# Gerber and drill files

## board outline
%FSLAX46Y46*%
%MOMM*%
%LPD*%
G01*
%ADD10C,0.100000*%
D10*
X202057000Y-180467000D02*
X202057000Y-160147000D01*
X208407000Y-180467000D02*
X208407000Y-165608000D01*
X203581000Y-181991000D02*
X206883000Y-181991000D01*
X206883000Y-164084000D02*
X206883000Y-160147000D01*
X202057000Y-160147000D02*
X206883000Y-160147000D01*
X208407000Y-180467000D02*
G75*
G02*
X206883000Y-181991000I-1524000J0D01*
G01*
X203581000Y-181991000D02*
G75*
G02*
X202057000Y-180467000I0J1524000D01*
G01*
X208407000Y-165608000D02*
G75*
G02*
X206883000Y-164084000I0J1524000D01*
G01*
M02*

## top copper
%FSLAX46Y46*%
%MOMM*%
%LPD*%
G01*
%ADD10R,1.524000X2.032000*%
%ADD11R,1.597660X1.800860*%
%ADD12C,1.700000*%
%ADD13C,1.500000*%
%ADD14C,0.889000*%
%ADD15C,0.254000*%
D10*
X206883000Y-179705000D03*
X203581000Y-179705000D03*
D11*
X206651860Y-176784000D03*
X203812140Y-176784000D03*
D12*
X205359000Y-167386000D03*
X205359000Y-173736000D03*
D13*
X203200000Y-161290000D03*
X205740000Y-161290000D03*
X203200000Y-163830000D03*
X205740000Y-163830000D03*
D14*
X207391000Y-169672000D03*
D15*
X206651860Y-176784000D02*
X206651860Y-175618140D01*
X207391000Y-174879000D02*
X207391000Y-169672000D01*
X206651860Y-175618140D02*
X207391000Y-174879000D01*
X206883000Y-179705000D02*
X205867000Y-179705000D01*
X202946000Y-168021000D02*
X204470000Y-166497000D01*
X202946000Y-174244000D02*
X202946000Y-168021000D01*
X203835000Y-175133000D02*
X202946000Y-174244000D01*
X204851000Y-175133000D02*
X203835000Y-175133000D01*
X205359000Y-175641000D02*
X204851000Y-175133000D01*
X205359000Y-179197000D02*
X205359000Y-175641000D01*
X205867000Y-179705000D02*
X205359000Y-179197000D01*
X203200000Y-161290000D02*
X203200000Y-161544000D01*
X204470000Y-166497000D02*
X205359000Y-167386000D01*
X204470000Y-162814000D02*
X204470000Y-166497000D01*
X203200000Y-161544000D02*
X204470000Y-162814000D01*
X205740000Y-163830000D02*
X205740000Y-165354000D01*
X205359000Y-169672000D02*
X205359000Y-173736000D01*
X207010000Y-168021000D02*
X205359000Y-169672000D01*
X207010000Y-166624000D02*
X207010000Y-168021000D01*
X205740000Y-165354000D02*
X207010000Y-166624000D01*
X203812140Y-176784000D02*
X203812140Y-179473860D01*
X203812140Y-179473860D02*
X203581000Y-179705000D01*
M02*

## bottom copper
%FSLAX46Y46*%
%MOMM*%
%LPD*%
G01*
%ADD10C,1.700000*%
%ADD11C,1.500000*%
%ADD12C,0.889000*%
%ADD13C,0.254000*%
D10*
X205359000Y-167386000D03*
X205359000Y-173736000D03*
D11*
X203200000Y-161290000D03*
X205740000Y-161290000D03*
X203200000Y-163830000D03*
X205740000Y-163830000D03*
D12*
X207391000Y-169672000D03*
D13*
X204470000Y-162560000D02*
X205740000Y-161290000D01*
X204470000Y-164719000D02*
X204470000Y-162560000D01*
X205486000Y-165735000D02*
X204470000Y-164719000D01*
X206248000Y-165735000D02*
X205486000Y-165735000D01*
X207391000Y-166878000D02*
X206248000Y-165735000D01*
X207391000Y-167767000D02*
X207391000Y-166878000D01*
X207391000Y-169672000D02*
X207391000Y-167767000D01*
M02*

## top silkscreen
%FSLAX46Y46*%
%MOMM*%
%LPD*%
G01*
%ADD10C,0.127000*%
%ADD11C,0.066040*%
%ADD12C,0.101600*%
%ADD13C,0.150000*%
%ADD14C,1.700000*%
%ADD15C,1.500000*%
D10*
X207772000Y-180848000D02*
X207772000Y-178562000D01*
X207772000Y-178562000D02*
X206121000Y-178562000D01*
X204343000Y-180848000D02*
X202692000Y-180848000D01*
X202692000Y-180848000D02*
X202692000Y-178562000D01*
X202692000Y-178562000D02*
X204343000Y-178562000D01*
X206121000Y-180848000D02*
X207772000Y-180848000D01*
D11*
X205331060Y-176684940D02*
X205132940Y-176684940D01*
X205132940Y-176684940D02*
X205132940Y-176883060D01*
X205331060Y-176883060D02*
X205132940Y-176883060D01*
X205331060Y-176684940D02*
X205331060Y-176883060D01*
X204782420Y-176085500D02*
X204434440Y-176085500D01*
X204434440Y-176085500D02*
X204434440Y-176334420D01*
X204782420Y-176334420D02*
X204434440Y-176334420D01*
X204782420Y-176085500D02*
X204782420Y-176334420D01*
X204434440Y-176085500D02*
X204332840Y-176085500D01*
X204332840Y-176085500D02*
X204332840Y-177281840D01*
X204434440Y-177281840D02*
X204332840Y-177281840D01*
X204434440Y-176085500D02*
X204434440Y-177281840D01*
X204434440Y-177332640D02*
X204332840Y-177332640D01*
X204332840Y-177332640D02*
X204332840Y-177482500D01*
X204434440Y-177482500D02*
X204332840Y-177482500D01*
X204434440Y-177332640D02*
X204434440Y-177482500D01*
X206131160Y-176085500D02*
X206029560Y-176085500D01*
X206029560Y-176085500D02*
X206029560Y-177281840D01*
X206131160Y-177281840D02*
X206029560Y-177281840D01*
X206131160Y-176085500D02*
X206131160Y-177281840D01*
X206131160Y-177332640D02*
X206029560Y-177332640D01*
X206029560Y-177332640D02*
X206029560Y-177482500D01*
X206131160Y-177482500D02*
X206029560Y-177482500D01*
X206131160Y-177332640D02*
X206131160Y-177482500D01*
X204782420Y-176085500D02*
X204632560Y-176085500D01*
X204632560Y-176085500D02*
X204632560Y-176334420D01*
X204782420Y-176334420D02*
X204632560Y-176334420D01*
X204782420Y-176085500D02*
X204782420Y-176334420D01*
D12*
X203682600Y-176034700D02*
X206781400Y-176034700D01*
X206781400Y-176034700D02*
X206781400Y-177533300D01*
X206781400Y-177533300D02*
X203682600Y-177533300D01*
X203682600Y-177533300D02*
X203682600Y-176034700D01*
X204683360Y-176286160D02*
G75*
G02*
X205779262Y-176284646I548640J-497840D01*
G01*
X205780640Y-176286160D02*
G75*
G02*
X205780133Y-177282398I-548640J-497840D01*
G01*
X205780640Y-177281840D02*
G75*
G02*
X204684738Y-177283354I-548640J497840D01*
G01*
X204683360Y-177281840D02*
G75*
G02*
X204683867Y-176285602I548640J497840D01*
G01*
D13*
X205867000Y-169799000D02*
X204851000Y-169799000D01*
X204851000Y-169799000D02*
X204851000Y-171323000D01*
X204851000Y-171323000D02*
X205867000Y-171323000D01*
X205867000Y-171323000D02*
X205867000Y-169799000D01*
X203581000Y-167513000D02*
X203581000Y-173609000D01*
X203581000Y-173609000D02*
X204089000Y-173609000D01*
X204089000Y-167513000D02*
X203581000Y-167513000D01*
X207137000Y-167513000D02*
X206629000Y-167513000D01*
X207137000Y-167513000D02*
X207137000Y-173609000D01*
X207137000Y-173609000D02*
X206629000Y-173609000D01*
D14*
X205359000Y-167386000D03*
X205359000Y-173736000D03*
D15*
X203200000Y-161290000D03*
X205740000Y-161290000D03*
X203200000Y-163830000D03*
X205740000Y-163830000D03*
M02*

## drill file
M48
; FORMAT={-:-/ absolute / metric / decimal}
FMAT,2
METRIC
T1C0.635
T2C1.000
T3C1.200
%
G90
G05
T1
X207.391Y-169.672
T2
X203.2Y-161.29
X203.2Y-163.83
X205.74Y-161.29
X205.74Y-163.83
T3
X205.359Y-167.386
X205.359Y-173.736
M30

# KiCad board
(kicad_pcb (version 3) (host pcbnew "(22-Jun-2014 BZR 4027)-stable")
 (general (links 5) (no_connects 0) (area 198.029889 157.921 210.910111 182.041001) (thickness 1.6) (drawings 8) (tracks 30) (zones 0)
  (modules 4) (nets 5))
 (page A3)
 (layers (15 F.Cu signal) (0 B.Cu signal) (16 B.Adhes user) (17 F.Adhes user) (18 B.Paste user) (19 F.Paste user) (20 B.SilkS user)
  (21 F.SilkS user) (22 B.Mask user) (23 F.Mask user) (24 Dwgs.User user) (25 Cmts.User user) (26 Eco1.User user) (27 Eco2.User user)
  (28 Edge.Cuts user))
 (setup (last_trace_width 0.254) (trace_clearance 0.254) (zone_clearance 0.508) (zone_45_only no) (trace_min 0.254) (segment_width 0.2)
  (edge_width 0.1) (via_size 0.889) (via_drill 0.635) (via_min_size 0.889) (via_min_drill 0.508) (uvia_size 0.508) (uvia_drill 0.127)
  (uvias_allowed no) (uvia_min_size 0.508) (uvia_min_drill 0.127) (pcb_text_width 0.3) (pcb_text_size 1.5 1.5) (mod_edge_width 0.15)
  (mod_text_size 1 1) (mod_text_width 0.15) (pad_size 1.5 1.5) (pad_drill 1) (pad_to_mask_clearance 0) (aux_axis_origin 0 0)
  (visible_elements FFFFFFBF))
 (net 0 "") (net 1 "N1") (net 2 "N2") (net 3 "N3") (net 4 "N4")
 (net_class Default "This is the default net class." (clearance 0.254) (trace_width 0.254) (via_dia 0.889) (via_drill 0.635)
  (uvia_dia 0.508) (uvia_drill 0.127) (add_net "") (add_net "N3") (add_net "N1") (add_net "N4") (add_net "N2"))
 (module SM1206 (layer F.Cu) (at 205.232 179.705 180)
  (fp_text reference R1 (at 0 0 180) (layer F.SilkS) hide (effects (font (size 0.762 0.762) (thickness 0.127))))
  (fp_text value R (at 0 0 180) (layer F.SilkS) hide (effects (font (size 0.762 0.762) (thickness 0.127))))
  (fp_line (start -2.54 -1.143) (end -2.54 1.143) (layer F.SilkS) (width 0.127))
  (fp_line (start -2.54 1.143) (end -0.889 1.143) (layer F.SilkS) (width 0.127))
  (fp_line (start 0.889 -1.143) (end 2.54 -1.143) (layer F.SilkS) (width 0.127))
  (fp_line (start 2.54 -1.143) (end 2.54 1.143) (layer F.SilkS) (width 0.127))
  (fp_line (start 2.54 1.143) (end 0.889 1.143) (layer F.SilkS) (width 0.127))
  (fp_line (start -0.889 -1.143) (end -2.54 -1.143) (layer F.SilkS) (width 0.127))
  (pad 1 smd rect (at -1.651 0 180) (size 1.524 2.032) (layers F.Cu F.Paste F.Mask) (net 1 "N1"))
  (pad 2 smd rect (at 1.651 0 180) (size 1.524 2.032) (layers F.Cu F.Paste F.Mask) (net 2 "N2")))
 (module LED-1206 (layer F.Cu) (at 205.232 176.784 180)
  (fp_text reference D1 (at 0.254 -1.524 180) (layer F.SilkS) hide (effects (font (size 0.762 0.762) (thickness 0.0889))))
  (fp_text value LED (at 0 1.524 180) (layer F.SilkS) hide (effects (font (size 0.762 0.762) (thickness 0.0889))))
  (fp_line (start -0.09906 0.09906) (end 0.09906 0.09906) (layer F.SilkS) (width 0.06604))
  (fp_line (start 0.09906 0.09906) (end 0.09906 -0.09906) (layer F.SilkS) (width 0.06604))
  (fp_line (start -0.09906 -0.09906) (end 0.09906 -0.09906) (layer F.SilkS) (width 0.06604))
  (fp_line (start -0.09906 0.09906) (end -0.09906 -0.09906) (layer F.SilkS) (width 0.06604))
  (fp_line (start 0.44958 0.6985) (end 0.79756 0.6985) (layer F.SilkS) (width 0.06604))
  (fp_line (start 0.79756 0.6985) (end 0.79756 0.44958) (layer F.SilkS) (width 0.06604))
  (fp_line (start 0.44958 0.44958) (end 0.79756 0.44958) (layer F.SilkS) (width 0.06604))
  (fp_line (start 0.44958 0.6985) (end 0.44958 0.44958) (layer F.SilkS) (width 0.06604))
  (fp_line (start 0.79756 0.6985) (end 0.89916 0.6985) (layer F.SilkS) (width 0.06604))
  (fp_line (start 0.89916 0.6985) (end 0.89916 -0.49784) (layer F.SilkS) (width 0.06604))
  (fp_line (start 0.79756 -0.49784) (end 0.89916 -0.49784) (layer F.SilkS) (width 0.06604))
  (fp_line (start 0.79756 0.6985) (end 0.79756 -0.49784) (layer F.SilkS) (width 0.06604))
  (fp_line (start 0.79756 -0.54864) (end 0.89916 -0.54864) (layer F.SilkS) (width 0.06604))
  (fp_line (start 0.89916 -0.54864) (end 0.89916 -0.6985) (layer F.SilkS) (width 0.06604))
  (fp_line (start 0.79756 -0.6985) (end 0.89916 -0.6985) (layer F.SilkS) (width 0.06604))
  (fp_line (start 0.79756 -0.54864) (end 0.79756 -0.6985) (layer F.SilkS) (width 0.06604))
  (fp_line (start -0.89916 0.6985) (end -0.79756 0.6985) (layer F.SilkS) (width 0.06604))
  (fp_line (start -0.79756 0.6985) (end -0.79756 -0.49784) (layer F.SilkS) (width 0.06604))
  (fp_line (start -0.89916 -0.49784) (end -0.79756 -0.49784) (layer F.SilkS) (width 0.06604))
  (fp_line (start -0.89916 0.6985) (end -0.89916 -0.49784) (layer F.SilkS) (width 0.06604))
  (fp_line (start -0.89916 -0.54864) (end -0.79756 -0.54864) (layer F.SilkS) (width 0.06604))
  (fp_line (start -0.79756 -0.54864) (end -0.79756 -0.6985) (layer F.SilkS) (width 0.06604))
  (fp_line (start -0.89916 -0.6985) (end -0.79756 -0.6985) (layer F.SilkS) (width 0.06604))
  (fp_line (start -0.89916 -0.54864) (end -0.89916 -0.6985) (layer F.SilkS) (width 0.06604))
  (fp_line (start 0.44958 0.6985) (end 0.59944 0.6985) (layer F.SilkS) (width 0.06604))
  (fp_line (start 0.59944 0.6985) (end 0.59944 0.44958) (layer F.SilkS) (width 0.06604))
  (fp_line (start 0.44958 0.44958) (end 0.59944 0.44958) (layer F.SilkS) (width 0.06604))
  (fp_line (start 0.44958 0.6985) (end 0.44958 0.44958) (layer F.SilkS) (width 0.06604))
  (fp_line (start 1.5494 0.7493) (end -1.5494 0.7493) (layer F.SilkS) (width 0.1016))
  (fp_line (start -1.5494 0.7493) (end -1.5494 -0.7493) (layer F.SilkS) (width 0.1016))
  (fp_line (start -1.5494 -0.7493) (end 1.5494 -0.7493) (layer F.SilkS) (width 0.1016))
  (fp_line (start 1.5494 -0.7493) (end 1.5494 0.7493) (layer F.SilkS) (width 0.1016))
  (fp_arc (start 0 0) (end 0.54864 0.49784) (angle 95.4) (layer F.SilkS) (width 0.1016))
  (fp_arc (start 0 0) (end -0.54864 0.49784) (angle 84.5) (layer F.SilkS) (width 0.1016))
  (fp_arc (start 0 0) (end -0.54864 -0.49784) (angle 95.4) (layer F.SilkS) (width 0.1016))
  (fp_arc (start 0 0) (end 0.54864 -0.49784) (angle 84.5) (layer F.SilkS) (width 0.1016))
  (pad 1 smd rect (at -1.41986 0 180) (size 1.59766 1.80086) (layers F.Cu F.Paste F.Mask) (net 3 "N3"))
  (pad 2 smd rect (at 1.41986 0 180) (size 1.59766 1.80086) (layers F.Cu F.Paste F.Mask) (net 2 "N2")))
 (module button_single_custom (layer F.Cu) (at 205.359 170.561 270)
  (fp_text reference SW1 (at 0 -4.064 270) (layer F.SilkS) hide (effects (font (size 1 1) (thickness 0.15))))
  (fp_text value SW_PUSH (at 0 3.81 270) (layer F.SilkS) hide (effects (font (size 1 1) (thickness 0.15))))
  (fp_line (start -0.762 -0.508) (end -0.762 0.508) (layer F.SilkS) (width 0.15))
  (fp_line (start -0.762 0.508) (end 0.762 0.508) (layer F.SilkS) (width 0.15))
  (fp_line (start 0.762 0.508) (end 0.762 -0.508) (layer F.SilkS) (width 0.15))
  (fp_line (start 0.762 -0.508) (end -0.762 -0.508) (layer F.SilkS) (width 0.15))
  (fp_line (start -3.048 1.778) (end 3.048 1.778) (layer F.SilkS) (width 0.15))
  (fp_line (start 3.048 1.778) (end 3.048 1.27) (layer F.SilkS) (width 0.15))
  (fp_line (start -3.048 1.27) (end -3.048 1.778) (layer F.SilkS) (width 0.15))
  (fp_line (start -3.048 -1.778) (end -3.048 -1.27) (layer F.SilkS) (width 0.15))
  (fp_line (start -3.048 -1.778) (end 3.048 -1.778) (layer F.SilkS) (width 0.15))
  (fp_line (start 3.048 -1.778) (end 3.048 -1.27) (layer F.SilkS) (width 0.15))
  (pad 1 thru_hole circle (at -3.175 0 270) (size 1.7 1.7) (drill 1.2) (layers *.Cu *.Mask F.SilkS) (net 1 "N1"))
  (pad 2 thru_hole circle (at 3.175 0 270) (size 1.7 1.7) (drill 1.2) (layers *.Cu *.Mask F.SilkS) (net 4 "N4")))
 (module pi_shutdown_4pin (layer F.Cu) (at 204.47 162.56)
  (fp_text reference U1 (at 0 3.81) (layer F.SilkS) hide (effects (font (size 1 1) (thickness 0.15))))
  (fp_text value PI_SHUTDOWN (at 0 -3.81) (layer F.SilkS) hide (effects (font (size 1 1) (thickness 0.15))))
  (pad 14 thru_hole circle (at -1.27 -1.27) (size 1.5 1.5) (drill 1) (layers *.Cu *.Mask F.SilkS) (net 1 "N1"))
  (pad 16 thru_hole circle (at 1.27 -1.27) (size 1.5 1.5) (drill 1) (layers *.Cu *.Mask F.SilkS) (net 3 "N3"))
  (pad 13 thru_hole circle (at -1.27 1.27) (size 1.5 1.5) (drill 1) (layers *.Cu *.Mask F.SilkS))
  (pad 15 thru_hole circle (at 1.27 1.27) (size 1.5 1.5) (drill 1) (layers *.Cu *.Mask F.SilkS) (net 4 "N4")))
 (gr_line (start 202.057 180.467) (end 202.057 160.147) (angle 90) (layer Edge.Cuts) (width 0.1))
 (gr_line (start 208.407 180.467) (end 208.407 165.608) (angle 90) (layer Edge.Cuts) (width 0.1))
 (gr_line (start 203.581 181.991) (end 206.883 181.991) (angle 90) (layer Edge.Cuts) (width 0.1))
 (gr_line (start 206.883 164.084) (end 206.883 160.147) (angle 90) (layer Edge.Cuts) (width 0.1))
 (gr_line (start 202.057 160.147) (end 206.883 160.147) (angle 90) (layer Edge.Cuts) (width 0.1))
 (gr_arc (start 206.883 180.467) (end 208.407 180.467) (angle 90) (layer Edge.Cuts) (width 0.1))
 (gr_arc (start 203.581 180.467) (end 203.581 181.991) (angle 90) (layer Edge.Cuts) (width 0.1))
 (gr_arc (start 208.407 164.084) (end 208.407 165.608) (angle 90) (layer Edge.Cuts) (width 0.1))
 (segment (start 206.65186 176.784) (end 206.65186 175.61814) (width 0.254) (layer F.Cu) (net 3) (status 400000))
 (segment (start 204.47 162.56) (end 205.74 161.29) (width 0.254) (layer B.Cu) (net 3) (status 800000))
 (segment (start 204.47 164.719) (end 204.47 162.56) (width 0.254) (layer B.Cu) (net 3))
 (segment (start 205.486 165.735) (end 204.47 164.719) (width 0.254) (layer B.Cu) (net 3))
 (segment (start 206.248 165.735) (end 205.486 165.735) (width 0.254) (layer B.Cu) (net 3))
 (segment (start 207.391 166.878) (end 206.248 165.735) (width 0.254) (layer B.Cu) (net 3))
 (segment (start 207.391 167.767) (end 207.391 166.878) (width 0.254) (layer B.Cu) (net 3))
 (segment (start 207.391 169.672) (end 207.391 167.767) (width 0.254) (layer B.Cu) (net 3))
 (segment (start 207.391 174.879) (end 207.391 169.672) (width 0.254) (layer F.Cu) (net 3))
 (segment (start 206.65186 175.61814) (end 207.391 174.879) (width 0.254) (layer F.Cu) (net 3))
 (segment (start 206.883 179.705) (end 205.867 179.705) (width 0.254) (layer F.Cu) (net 1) (status 400000))
 (segment (start 202.946 168.021) (end 204.47 166.497) (width 0.254) (layer F.Cu) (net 1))
 (segment (start 202.946 174.244) (end 202.946 168.021) (width 0.254) (layer F.Cu) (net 1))
 (segment (start 203.835 175.133) (end 202.946 174.244) (width 0.254) (layer F.Cu) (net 1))
 (segment (start 204.851 175.133) (end 203.835 175.133) (width 0.254) (layer F.Cu) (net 1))
 (segment (start 205.359 175.641) (end 204.851 175.133) (width 0.254) (layer F.Cu) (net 1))
 (segment (start 205.359 179.197) (end 205.359 175.641) (width 0.254) (layer F.Cu) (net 1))
 (segment (start 205.867 179.705) (end 205.359 179.197) (width 0.254) (layer F.Cu) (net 1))
 (segment (start 203.2 161.29) (end 203.2 161.544) (width 0.254) (layer F.Cu) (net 1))
 (segment (start 204.47 166.497) (end 205.359 167.386) (width 0.254) (layer F.Cu) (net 1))
 (segment (start 204.47 162.814) (end 204.47 166.497) (width 0.254) (layer F.Cu) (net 1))
 (segment (start 203.2 161.544) (end 204.47 162.814) (width 0.254) (layer F.Cu) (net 1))
 (segment (start 205.74 163.83) (end 205.74 165.354) (width 0.254) (layer F.Cu) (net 4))
 (segment (start 205.359 169.672) (end 205.359 173.736) (width 0.254) (layer F.Cu) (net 4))
 (segment (start 207.01 168.021) (end 205.359 169.672) (width 0.254) (layer F.Cu) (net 4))
 (segment (start 207.01 166.624) (end 207.01 168.021) (width 0.254) (layer F.Cu) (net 4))
 (segment (start 205.74 165.354) (end 207.01 166.624) (width 0.254) (layer F.Cu) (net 4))
 (segment (start 203.81214 176.784) (end 203.81214 179.47386) (width 0.254) (layer F.Cu) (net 2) (status C00000))
 (segment (start 203.81214 179.47386) (end 203.581 179.705) (width 0.254) (layer F.Cu) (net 2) (status C00000))
 (via (at 207.391 169.672) (size 0.889) (layers F.Cu B.Cu) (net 3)))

